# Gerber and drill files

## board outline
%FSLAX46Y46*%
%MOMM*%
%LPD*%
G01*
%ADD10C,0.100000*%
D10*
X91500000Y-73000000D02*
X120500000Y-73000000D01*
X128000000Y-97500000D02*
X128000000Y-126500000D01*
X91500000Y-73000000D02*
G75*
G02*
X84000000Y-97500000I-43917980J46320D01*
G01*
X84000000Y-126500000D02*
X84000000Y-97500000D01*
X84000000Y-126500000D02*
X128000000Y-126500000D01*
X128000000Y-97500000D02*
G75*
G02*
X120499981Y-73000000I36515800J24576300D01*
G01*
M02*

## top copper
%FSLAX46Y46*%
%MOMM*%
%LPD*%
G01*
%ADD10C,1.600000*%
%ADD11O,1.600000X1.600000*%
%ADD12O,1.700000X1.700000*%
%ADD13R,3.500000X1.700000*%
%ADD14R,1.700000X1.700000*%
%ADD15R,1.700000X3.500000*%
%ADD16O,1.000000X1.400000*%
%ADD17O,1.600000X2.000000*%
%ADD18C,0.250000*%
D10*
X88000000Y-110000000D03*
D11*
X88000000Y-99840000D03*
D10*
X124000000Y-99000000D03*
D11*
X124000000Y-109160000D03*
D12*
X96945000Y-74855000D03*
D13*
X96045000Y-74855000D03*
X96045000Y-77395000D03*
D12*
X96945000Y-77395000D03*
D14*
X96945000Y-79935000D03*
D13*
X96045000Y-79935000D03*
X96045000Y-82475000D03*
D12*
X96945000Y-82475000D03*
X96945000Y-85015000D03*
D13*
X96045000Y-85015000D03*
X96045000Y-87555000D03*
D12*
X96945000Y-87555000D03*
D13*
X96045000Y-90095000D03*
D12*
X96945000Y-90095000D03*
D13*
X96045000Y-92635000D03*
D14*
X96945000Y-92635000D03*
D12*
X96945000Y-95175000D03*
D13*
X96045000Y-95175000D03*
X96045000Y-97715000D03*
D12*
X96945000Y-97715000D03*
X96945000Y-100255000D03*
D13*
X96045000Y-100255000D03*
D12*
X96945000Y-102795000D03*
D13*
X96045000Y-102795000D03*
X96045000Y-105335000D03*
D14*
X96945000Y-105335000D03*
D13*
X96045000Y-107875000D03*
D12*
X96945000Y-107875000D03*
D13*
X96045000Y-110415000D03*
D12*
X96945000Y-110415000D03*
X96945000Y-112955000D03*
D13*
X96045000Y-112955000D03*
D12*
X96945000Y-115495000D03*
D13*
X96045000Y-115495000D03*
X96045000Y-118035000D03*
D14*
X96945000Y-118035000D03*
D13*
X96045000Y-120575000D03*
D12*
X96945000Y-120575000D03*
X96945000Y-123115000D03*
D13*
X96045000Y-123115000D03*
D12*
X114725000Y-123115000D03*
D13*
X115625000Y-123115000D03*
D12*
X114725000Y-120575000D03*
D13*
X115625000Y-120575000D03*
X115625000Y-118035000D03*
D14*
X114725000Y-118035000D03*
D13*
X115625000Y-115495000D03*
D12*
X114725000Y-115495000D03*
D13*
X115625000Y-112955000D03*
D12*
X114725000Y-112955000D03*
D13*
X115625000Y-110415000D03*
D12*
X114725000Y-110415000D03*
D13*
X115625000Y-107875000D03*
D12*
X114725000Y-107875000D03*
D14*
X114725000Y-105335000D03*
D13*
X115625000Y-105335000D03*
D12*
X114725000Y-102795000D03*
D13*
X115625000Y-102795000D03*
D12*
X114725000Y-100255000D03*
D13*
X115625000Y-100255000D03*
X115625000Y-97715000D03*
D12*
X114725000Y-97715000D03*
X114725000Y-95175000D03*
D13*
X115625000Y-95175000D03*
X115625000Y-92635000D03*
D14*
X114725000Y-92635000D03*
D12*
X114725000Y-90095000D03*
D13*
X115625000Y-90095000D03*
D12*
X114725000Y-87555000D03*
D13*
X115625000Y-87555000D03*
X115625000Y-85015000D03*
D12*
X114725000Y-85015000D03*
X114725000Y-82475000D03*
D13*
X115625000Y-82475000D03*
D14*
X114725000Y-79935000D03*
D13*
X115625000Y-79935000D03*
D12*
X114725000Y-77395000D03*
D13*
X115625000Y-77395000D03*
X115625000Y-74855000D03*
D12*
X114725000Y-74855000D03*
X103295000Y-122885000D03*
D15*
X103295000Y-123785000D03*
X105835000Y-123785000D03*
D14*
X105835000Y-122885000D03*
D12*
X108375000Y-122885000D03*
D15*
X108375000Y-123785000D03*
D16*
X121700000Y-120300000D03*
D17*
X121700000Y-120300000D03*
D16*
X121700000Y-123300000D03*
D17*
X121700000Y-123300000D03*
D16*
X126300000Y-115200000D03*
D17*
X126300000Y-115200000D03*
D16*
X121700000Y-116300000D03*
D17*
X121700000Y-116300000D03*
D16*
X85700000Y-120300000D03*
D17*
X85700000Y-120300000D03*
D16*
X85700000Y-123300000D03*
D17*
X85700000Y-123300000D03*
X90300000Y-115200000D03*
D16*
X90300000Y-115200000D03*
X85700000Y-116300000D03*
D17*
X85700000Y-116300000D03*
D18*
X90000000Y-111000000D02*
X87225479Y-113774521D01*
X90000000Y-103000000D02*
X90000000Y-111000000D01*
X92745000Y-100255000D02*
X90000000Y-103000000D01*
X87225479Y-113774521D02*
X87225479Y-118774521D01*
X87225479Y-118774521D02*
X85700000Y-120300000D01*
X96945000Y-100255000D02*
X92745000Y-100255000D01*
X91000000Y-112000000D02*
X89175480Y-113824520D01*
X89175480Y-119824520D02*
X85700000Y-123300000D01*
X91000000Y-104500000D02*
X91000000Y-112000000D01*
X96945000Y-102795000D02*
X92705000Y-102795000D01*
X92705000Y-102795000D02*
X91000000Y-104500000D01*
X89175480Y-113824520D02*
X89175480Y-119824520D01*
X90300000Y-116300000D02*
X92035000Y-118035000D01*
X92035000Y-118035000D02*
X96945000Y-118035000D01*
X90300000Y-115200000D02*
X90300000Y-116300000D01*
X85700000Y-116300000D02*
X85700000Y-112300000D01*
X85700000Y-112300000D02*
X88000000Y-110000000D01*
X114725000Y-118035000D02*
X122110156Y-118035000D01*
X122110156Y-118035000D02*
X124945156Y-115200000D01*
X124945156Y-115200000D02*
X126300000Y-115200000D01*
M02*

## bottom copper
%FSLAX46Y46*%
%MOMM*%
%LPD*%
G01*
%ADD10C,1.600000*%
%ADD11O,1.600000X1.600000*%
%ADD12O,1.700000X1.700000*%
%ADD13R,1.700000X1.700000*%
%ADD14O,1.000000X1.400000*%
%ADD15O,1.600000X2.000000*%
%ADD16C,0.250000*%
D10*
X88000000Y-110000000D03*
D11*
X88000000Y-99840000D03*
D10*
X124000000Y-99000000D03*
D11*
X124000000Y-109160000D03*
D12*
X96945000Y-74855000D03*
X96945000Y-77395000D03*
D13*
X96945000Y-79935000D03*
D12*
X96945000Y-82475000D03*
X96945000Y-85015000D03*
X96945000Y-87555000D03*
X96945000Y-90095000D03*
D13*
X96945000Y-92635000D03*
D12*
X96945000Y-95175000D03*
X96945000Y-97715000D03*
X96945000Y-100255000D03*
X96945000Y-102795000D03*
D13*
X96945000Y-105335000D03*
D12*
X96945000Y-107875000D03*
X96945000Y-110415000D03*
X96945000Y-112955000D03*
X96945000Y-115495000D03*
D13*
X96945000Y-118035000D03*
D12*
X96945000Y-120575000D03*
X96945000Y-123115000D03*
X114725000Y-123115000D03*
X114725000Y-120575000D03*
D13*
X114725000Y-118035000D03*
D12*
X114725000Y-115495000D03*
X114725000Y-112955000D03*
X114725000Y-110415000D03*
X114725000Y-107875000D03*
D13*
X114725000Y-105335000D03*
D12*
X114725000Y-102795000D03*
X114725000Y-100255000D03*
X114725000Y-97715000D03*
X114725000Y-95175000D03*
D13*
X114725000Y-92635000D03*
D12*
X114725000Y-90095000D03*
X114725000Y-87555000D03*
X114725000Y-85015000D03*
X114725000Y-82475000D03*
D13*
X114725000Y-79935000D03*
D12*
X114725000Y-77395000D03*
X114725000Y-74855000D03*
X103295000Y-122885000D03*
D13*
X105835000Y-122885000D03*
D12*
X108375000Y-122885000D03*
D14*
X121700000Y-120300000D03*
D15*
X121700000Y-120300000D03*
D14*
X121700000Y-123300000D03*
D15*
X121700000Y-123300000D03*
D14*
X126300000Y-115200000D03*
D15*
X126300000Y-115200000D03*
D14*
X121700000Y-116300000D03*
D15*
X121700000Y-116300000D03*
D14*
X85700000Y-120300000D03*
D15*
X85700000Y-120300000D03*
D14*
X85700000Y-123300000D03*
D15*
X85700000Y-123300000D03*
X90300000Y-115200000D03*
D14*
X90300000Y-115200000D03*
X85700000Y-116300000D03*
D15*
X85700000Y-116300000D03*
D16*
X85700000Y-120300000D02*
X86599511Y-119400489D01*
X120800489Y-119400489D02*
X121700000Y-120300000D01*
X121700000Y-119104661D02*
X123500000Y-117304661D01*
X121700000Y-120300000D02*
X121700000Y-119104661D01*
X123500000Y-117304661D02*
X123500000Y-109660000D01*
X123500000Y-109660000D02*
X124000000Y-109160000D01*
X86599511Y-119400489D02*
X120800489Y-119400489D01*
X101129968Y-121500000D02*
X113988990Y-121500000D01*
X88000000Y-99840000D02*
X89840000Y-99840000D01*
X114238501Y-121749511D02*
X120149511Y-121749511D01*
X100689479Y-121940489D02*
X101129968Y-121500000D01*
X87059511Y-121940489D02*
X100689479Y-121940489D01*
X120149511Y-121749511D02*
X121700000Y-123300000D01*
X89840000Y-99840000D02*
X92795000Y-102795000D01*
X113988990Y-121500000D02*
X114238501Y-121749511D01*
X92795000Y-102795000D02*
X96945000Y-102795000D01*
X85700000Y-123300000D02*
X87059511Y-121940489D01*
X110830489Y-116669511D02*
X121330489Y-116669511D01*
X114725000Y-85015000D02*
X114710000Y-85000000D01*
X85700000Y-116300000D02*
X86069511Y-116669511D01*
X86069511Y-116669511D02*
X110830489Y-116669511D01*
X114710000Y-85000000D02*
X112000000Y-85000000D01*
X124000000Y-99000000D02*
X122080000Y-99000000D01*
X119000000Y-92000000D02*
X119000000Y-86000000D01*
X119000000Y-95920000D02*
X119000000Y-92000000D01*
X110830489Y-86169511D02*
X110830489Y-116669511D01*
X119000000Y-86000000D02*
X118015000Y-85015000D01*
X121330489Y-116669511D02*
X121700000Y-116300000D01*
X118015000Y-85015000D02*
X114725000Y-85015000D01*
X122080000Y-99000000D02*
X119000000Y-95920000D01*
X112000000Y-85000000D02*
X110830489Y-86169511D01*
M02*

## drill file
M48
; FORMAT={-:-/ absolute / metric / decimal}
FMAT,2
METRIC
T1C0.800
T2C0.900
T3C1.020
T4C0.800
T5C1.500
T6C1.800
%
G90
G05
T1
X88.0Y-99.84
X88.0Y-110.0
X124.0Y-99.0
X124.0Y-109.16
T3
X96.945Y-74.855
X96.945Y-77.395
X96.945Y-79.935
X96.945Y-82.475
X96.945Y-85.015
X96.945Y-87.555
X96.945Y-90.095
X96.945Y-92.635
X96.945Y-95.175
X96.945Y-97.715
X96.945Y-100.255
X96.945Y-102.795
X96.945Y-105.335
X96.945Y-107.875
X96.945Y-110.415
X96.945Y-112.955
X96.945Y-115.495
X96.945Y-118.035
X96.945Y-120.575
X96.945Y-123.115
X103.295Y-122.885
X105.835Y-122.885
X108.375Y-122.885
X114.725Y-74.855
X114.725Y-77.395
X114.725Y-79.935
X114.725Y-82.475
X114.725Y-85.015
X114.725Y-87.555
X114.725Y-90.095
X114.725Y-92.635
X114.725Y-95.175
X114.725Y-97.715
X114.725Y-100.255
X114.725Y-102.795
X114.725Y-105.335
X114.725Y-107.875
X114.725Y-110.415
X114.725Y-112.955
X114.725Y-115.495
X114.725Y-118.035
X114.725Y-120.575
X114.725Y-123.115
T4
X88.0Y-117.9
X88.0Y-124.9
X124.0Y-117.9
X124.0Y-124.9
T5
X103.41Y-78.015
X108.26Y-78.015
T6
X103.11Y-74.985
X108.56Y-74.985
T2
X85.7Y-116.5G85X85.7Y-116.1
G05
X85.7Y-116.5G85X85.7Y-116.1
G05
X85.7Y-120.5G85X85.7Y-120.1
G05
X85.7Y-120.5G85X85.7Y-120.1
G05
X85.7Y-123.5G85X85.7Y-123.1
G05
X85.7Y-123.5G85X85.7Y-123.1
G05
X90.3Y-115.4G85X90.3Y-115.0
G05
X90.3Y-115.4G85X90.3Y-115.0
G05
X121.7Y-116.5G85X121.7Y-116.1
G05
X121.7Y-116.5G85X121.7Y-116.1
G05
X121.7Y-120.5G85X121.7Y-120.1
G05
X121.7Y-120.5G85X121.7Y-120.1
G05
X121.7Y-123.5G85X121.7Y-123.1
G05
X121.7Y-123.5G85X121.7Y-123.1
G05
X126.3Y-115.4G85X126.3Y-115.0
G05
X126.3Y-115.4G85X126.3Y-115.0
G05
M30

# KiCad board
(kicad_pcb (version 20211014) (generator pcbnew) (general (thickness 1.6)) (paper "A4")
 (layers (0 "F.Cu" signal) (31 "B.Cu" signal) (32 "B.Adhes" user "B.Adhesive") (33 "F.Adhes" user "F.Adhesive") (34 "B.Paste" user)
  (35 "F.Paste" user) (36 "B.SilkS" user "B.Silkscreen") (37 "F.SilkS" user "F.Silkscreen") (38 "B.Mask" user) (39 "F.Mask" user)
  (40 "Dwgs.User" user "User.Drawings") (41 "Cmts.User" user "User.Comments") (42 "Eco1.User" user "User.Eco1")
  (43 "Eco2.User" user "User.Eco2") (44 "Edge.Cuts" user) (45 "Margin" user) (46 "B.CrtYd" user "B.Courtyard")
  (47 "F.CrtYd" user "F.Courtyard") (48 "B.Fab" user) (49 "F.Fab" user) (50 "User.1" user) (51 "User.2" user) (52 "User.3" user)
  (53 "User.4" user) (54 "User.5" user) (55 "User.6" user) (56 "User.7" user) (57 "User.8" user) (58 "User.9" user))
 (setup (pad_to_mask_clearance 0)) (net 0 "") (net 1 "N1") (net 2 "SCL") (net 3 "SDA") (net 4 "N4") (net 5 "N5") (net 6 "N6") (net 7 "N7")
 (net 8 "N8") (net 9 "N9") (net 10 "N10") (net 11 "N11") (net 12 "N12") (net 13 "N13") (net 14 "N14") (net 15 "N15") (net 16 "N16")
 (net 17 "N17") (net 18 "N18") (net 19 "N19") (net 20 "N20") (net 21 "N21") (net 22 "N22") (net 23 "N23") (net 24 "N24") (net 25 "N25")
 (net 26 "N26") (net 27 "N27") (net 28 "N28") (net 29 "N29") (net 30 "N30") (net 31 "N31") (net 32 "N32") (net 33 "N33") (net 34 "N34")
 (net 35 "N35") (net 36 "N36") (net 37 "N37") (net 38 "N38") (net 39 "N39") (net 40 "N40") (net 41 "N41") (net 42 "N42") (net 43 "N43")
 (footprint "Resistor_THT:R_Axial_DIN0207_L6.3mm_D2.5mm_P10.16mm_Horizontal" (layer "F.Cu") (at 88 110 90)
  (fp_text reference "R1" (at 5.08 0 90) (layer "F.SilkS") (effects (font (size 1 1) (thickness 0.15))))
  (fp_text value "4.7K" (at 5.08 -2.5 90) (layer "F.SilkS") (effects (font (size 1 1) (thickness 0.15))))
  (pad "1" thru_hole circle (at 0 0 90) (size 1.6 1.6) (drill 0.8) (layers *.Cu *.Mask) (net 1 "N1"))
  (pad "2" thru_hole oval (at 10.16 0 90) (size 1.6 1.6) (drill 0.8) (layers *.Cu *.Mask) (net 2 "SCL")))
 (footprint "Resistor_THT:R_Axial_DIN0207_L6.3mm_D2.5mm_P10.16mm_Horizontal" (layer "F.Cu") (at 124 99 -90)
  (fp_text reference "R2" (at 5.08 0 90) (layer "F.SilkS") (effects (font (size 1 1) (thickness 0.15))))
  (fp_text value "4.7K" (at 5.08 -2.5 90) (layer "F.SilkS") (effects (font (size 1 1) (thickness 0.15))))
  (pad "1" thru_hole circle (at 0 0 270) (size 1.6 1.6) (drill 0.8) (layers *.Cu *.Mask) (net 1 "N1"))
  (pad "2" thru_hole oval (at 10.16 0 270) (size 1.6 1.6) (drill 0.8) (layers *.Cu *.Mask) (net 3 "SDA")))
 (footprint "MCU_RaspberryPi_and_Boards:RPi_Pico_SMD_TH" (layer "F.Cu") (at 105.835 98.985)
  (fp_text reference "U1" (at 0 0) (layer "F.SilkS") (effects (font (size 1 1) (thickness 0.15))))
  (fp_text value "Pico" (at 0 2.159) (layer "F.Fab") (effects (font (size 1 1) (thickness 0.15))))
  (pad "" np_thru_hole oval (at 2.725 -24) (size 1.8 1.8) (drill 1.8) (layers *.Cu *.Mask))
  (pad "" np_thru_hole oval (at -2.725 -24) (size 1.8 1.8) (drill 1.8) (layers *.Cu *.Mask))
  (pad "" np_thru_hole oval (at -2.425 -20.97) (size 1.5 1.5) (drill 1.5) (layers *.Cu *.Mask))
  (pad "" np_thru_hole oval (at 2.425 -20.97) (size 1.5 1.5) (drill 1.5) (layers *.Cu *.Mask))
  (pad "1" thru_hole oval (at -8.89 -24.13) (size 1.7 1.7) (drill 1.02) (layers *.Cu *.Mask) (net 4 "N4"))
  (pad "1" smd rect (at -8.89 -24.13) (size 3.5 1.7) (drill (offset -0.9 0)) (layers "F.Cu" "F.Mask") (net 4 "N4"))
  (pad "2" smd rect (at -8.89 -21.59) (size 3.5 1.7) (drill (offset -0.9 0)) (layers "F.Cu" "F.Mask") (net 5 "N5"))
  (pad "2" thru_hole oval (at -8.89 -21.59) (size 1.7 1.7) (drill 1.02) (layers *.Cu *.Mask) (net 5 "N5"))
  (pad "3" thru_hole rect (at -8.89 -19.05) (size 1.7 1.7) (drill 1.02) (layers *.Cu *.Mask) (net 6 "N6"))
  (pad "3" smd rect (at -8.89 -19.05) (size 3.5 1.7) (drill (offset -0.9 0)) (layers "F.Cu" "F.Mask") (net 6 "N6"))
  (pad "4" smd rect (at -8.89 -16.51) (size 3.5 1.7) (drill (offset -0.9 0)) (layers "F.Cu" "F.Mask") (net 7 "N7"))
  (pad "4" thru_hole oval (at -8.89 -16.51) (size 1.7 1.7) (drill 1.02) (layers *.Cu *.Mask) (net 7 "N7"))
  (pad "5" thru_hole oval (at -8.89 -13.97) (size 1.7 1.7) (drill 1.02) (layers *.Cu *.Mask) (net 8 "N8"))
  (pad "5" smd rect (at -8.89 -13.97) (size 3.5 1.7) (drill (offset -0.9 0)) (layers "F.Cu" "F.Mask") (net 8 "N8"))
  (pad "6" smd rect (at -8.89 -11.43) (size 3.5 1.7) (drill (offset -0.9 0)) (layers "F.Cu" "F.Mask") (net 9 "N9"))
  (pad "6" thru_hole oval (at -8.89 -11.43) (size 1.7 1.7) (drill 1.02) (layers *.Cu *.Mask) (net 9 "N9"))
  (pad "7" smd rect (at -8.89 -8.89) (size 3.5 1.7) (drill (offset -0.9 0)) (layers "F.Cu" "F.Mask") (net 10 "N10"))
  (pad "7" thru_hole oval (at -8.89 -8.89) (size 1.7 1.7) (drill 1.02) (layers *.Cu *.Mask) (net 10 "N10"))
  (pad "8" smd rect (at -8.89 -6.35) (size 3.5 1.7) (drill (offset -0.9 0)) (layers "F.Cu" "F.Mask") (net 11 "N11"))
  (pad "8" thru_hole rect (at -8.89 -6.35) (size 1.7 1.7) (drill 1.02) (layers *.Cu *.Mask) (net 11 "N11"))
  (pad "9" thru_hole oval (at -8.89 -3.81) (size 1.7 1.7) (drill 1.02) (layers *.Cu *.Mask) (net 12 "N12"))
  (pad "9" smd rect (at -8.89 -3.81) (size 3.5 1.7) (drill (offset -0.9 0)) (layers "F.Cu" "F.Mask") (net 12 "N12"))
  (pad "10" smd rect (at -8.89 -1.27) (size 3.5 1.7) (drill (offset -0.9 0)) (layers "F.Cu" "F.Mask") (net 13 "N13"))
  (pad "10" thru_hole oval (at -8.89 -1.27) (size 1.7 1.7) (drill 1.02) (layers *.Cu *.Mask) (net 13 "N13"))
  (pad "11" thru_hole oval (at -8.89 1.27) (size 1.7 1.7) (drill 1.02) (layers *.Cu *.Mask) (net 3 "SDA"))
  (pad "11" smd rect (at -8.89 1.27) (size 3.5 1.7) (drill (offset -0.9 0)) (layers "F.Cu" "F.Mask") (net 3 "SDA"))
  (pad "12" thru_hole oval (at -8.89 3.81) (size 1.7 1.7) (drill 1.02) (layers *.Cu *.Mask) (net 2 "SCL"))
  (pad "12" smd rect (at -8.89 3.81) (size 3.5 1.7) (drill (offset -0.9 0)) (layers "F.Cu" "F.Mask") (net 2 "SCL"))
  (pad "13" smd rect (at -8.89 6.35) (size 3.5 1.7) (drill (offset -0.9 0)) (layers "F.Cu" "F.Mask") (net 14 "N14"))
  (pad "13" thru_hole rect (at -8.89 6.35) (size 1.7 1.7) (drill 1.02) (layers *.Cu *.Mask) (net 14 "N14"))
  (pad "14" smd rect (at -8.89 8.89) (size 3.5 1.7) (drill (offset -0.9 0)) (layers "F.Cu" "F.Mask") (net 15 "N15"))
  (pad "14" thru_hole oval (at -8.89 8.89) (size 1.7 1.7) (drill 1.02) (layers *.Cu *.Mask) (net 15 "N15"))
  (pad "15" smd rect (at -8.89 11.43) (size 3.5 1.7) (drill (offset -0.9 0)) (layers "F.Cu" "F.Mask") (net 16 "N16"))
  (pad "15" thru_hole oval (at -8.89 11.43) (size 1.7 1.7) (drill 1.02) (layers *.Cu *.Mask) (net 16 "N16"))
  (pad "16" thru_hole oval (at -8.89 13.97) (size 1.7 1.7) (drill 1.02) (layers *.Cu *.Mask) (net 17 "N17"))
  (pad "16" smd rect (at -8.89 13.97) (size 3.5 1.7) (drill (offset -0.9 0)) (layers "F.Cu" "F.Mask") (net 17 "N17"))
  (pad "17" thru_hole oval (at -8.89 16.51) (size 1.7 1.7) (drill 1.02) (layers *.Cu *.Mask) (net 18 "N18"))
  (pad "17" smd rect (at -8.89 16.51) (size 3.5 1.7) (drill (offset -0.9 0)) (layers "F.Cu" "F.Mask") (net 18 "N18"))
  (pad "18" smd rect (at -8.89 19.05) (size 3.5 1.7) (drill (offset -0.9 0)) (layers "F.Cu" "F.Mask") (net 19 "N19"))
  (pad "18" thru_hole rect (at -8.89 19.05) (size 1.7 1.7) (drill 1.02) (layers *.Cu *.Mask) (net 19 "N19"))
  (pad "19" smd rect (at -8.89 21.59) (size 3.5 1.7) (drill (offset -0.9 0)) (layers "F.Cu" "F.Mask") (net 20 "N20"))
  (pad "19" thru_hole oval (at -8.89 21.59) (size 1.7 1.7) (drill 1.02) (layers *.Cu *.Mask) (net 20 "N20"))
  (pad "20" thru_hole oval (at -8.89 24.13) (size 1.7 1.7) (drill 1.02) (layers *.Cu *.Mask) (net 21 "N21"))
  (pad "20" smd rect (at -8.89 24.13) (size 3.5 1.7) (drill (offset -0.9 0)) (layers "F.Cu" "F.Mask") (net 21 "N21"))
  (pad "21" thru_hole oval (at 8.89 24.13) (size 1.7 1.7) (drill 1.02) (layers *.Cu *.Mask) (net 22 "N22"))
  (pad "21" smd rect (at 8.89 24.13) (size 3.5 1.7) (drill (offset 0.9 0)) (layers "F.Cu" "F.Mask") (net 22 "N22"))
  (pad "22" thru_hole oval (at 8.89 21.59) (size 1.7 1.7) (drill 1.02) (layers *.Cu *.Mask) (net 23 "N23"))
  (pad "22" smd rect (at 8.89 21.59) (size 3.5 1.7) (drill (offset 0.9 0)) (layers "F.Cu" "F.Mask") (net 23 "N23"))
  (pad "23" smd rect (at 8.89 19.05) (size 3.5 1.7) (drill (offset 0.9 0)) (layers "F.Cu" "F.Mask") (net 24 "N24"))
  (pad "23" thru_hole rect (at 8.89 19.05) (size 1.7 1.7) (drill 1.02) (layers *.Cu *.Mask) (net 24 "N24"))
  (pad "24" smd rect (at 8.89 16.51) (size 3.5 1.7) (drill (offset 0.9 0)) (layers "F.Cu" "F.Mask") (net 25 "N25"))
  (pad "24" thru_hole oval (at 8.89 16.51) (size 1.7 1.7) (drill 1.02) (layers *.Cu *.Mask) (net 25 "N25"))
  (pad "25" smd rect (at 8.89 13.97) (size 3.5 1.7) (drill (offset 0.9 0)) (layers "F.Cu" "F.Mask") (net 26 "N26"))
  (pad "25" thru_hole oval (at 8.89 13.97) (size 1.7 1.7) (drill 1.02) (layers *.Cu *.Mask) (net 26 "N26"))
  (pad "26" smd rect (at 8.89 11.43) (size 3.5 1.7) (drill (offset 0.9 0)) (layers "F.Cu" "F.Mask") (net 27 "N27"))
  (pad "26" thru_hole oval (at 8.89 11.43) (size 1.7 1.7) (drill 1.02) (layers *.Cu *.Mask) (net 27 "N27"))
  (pad "27" smd rect (at 8.89 8.89) (size 3.5 1.7) (drill (offset 0.9 0)) (layers "F.Cu" "F.Mask") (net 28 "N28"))
  (pad "27" thru_hole oval (at 8.89 8.89) (size 1.7 1.7) (drill 1.02) (layers *.Cu *.Mask) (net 28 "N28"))
  (pad "28" thru_hole rect (at 8.89 6.35) (size 1.7 1.7) (drill 1.02) (layers *.Cu *.Mask) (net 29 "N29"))
  (pad "28" smd rect (at 8.89 6.35) (size 3.5 1.7) (drill (offset 0.9 0)) (layers "F.Cu" "F.Mask") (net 29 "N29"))
  (pad "29" thru_hole oval (at 8.89 3.81) (size 1.7 1.7) (drill 1.02) (layers *.Cu *.Mask) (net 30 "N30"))
  (pad "29" smd rect (at 8.89 3.81) (size 3.5 1.7) (drill (offset 0.9 0)) (layers "F.Cu" "F.Mask") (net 30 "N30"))
  (pad "30" thru_hole oval (at 8.89 1.27) (size 1.7 1.7) (drill 1.02) (layers *.Cu *.Mask) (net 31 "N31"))
  (pad "30" smd rect (at 8.89 1.27) (size 3.5 1.7) (drill (offset 0.9 0)) (layers "F.Cu" "F.Mask") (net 31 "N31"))
  (pad "31" smd rect (at 8.89 -1.27) (size 3.5 1.7) (drill (offset 0.9 0)) (layers "F.Cu" "F.Mask") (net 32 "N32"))
  (pad "31" thru_hole oval (at 8.89 -1.27) (size 1.7 1.7) (drill 1.02) (layers *.Cu *.Mask) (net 32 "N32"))
  (pad "32" thru_hole oval (at 8.89 -3.81) (size 1.7 1.7) (drill 1.02) (layers *.Cu *.Mask) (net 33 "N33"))
  (pad "32" smd rect (at 8.89 -3.81) (size 3.5 1.7) (drill (offset 0.9 0)) (layers "F.Cu" "F.Mask") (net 33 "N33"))
  (pad "33" smd rect (at 8.89 -6.35) (size 3.5 1.7) (drill (offset 0.9 0)) (layers "F.Cu" "F.Mask") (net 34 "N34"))
  (pad "33" thru_hole rect (at 8.89 -6.35) (size 1.7 1.7) (drill 1.02) (layers *.Cu *.Mask) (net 34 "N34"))
  (pad "34" thru_hole oval (at 8.89 -8.89) (size 1.7 1.7) (drill 1.02) (layers *.Cu *.Mask) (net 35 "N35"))
  (pad "34" smd rect (at 8.89 -8.89) (size 3.5 1.7) (drill (offset 0.9 0)) (layers "F.Cu" "F.Mask") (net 35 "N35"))
  (pad "35" thru_hole oval (at 8.89 -11.43) (size 1.7 1.7) (drill 1.02) (layers *.Cu *.Mask) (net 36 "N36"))
  (pad "35" smd rect (at 8.89 -11.43) (size 3.5 1.7) (drill (offset 0.9 0)) (layers "F.Cu" "F.Mask") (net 36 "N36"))
  (pad "36" smd rect (at 8.89 -13.97) (size 3.5 1.7) (drill (offset 0.9 0)) (layers "F.Cu" "F.Mask") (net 1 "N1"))
  (pad "36" thru_hole oval (at 8.89 -13.97) (size 1.7 1.7) (drill 1.02) (layers *.Cu *.Mask) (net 1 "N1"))
  (pad "37" thru_hole oval (at 8.89 -16.51) (size 1.7 1.7) (drill 1.02) (layers *.Cu *.Mask) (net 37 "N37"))
  (pad "37" smd rect (at 8.89 -16.51) (size 3.5 1.7) (drill (offset 0.9 0)) (layers "F.Cu" "F.Mask") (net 37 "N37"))
  (pad "38" thru_hole rect (at 8.89 -19.05) (size 1.7 1.7) (drill 1.02) (layers *.Cu *.Mask) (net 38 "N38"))
  (pad "38" smd rect (at 8.89 -19.05) (size 3.5 1.7) (drill (offset 0.9 0)) (layers "F.Cu" "F.Mask") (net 38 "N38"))
  (pad "39" thru_hole oval (at 8.89 -21.59) (size 1.7 1.7) (drill 1.02) (layers *.Cu *.Mask) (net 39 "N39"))
  (pad "39" smd rect (at 8.89 -21.59) (size 3.5 1.7) (drill (offset 0.9 0)) (layers "F.Cu" "F.Mask") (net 39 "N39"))
  (pad "40" smd rect (at 8.89 -24.13) (size 3.5 1.7) (drill (offset 0.9 0)) (layers "F.Cu" "F.Mask") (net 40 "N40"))
  (pad "40" thru_hole oval (at 8.89 -24.13) (size 1.7 1.7) (drill 1.02) (layers *.Cu *.Mask) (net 40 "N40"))
  (pad "41" thru_hole oval (at -2.54 23.9) (size 1.7 1.7) (drill 1.02) (layers *.Cu *.Mask) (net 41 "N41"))
  (pad "41" smd rect (at -2.54 23.9 90) (size 3.5 1.7) (drill (offset -0.9 0)) (layers "F.Cu" "F.Mask") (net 41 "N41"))
  (pad "42" smd rect (at 0 23.9 90) (size 3.5 1.7) (drill (offset -0.9 0)) (layers "F.Cu" "F.Mask") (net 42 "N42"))
  (pad "42" thru_hole rect (at 0 23.9) (size 1.7 1.7) (drill 1.02) (layers *.Cu *.Mask) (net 42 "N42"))
  (pad "43" thru_hole oval (at 2.54 23.9) (size 1.7 1.7) (drill 1.02) (layers *.Cu *.Mask) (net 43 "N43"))
  (pad "43" smd rect (at 2.54 23.9 90) (size 3.5 1.7) (drill (offset -0.9 0)) (layers "F.Cu" "F.Mask") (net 43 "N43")))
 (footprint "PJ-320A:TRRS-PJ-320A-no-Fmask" (layer "F.Cu") (at 124 126.5 180)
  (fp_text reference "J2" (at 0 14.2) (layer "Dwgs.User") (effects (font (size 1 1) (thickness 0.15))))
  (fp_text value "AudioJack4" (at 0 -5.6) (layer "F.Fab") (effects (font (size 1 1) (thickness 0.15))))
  (pad "" np_thru_hole circle (at 0 1.6 180) (size 0.8 0.8) (drill 0.8) (layers *.Cu *.Mask))
  (pad "" np_thru_hole circle (at 0 8.6 180) (size 0.8 0.8) (drill 0.8) (layers *.Cu *.Mask))
  (pad "R1" thru_hole oval (at 2.3 6.2 180) (size 1 1.4) (drill oval 0.9 1.3) (layers *.Cu "F.Mask") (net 3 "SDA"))
  (pad "R1" thru_hole oval (at 2.3 6.2 180) (size 1.6 2) (drill oval 0.9 1.3) (layers *.Cu "B.Mask") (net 3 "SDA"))
  (pad "R2" thru_hole oval (at 2.3 3.2 180) (size 1 1.4) (drill oval 0.9 1.3) (layers *.Cu "F.Mask") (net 2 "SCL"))
  (pad "R2" thru_hole oval (at 2.3 3.2 180) (size 1.6 2) (drill oval 0.9 1.3) (layers *.Cu "B.Mask") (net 2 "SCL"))
  (pad "S" thru_hole oval (at -2.3 11.3 180) (size 1 1.4) (drill oval 0.9 1.3) (layers *.Cu "F.Mask") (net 24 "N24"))
  (pad "S" thru_hole oval (at -2.3 11.3 180) (size 1.6 2) (drill oval 0.9 1.3) (layers *.Cu "B.Mask") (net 24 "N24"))
  (pad "T" thru_hole oval (at 2.3 10.2 180) (size 1 1.4) (drill oval 0.9 1.3) (layers *.Cu "F.Mask") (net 1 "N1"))
  (pad "T" thru_hole oval (at 2.3 10.2 180) (size 1.6 2) (drill oval 0.9 1.3) (layers *.Cu "B.Mask") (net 1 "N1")))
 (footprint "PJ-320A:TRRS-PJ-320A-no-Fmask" (layer "F.Cu") (at 88 126.5 180)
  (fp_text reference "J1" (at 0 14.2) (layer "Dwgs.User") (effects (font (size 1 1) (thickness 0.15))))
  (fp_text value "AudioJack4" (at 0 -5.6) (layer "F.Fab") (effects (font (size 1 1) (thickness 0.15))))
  (pad "" np_thru_hole circle (at 0 8.6 180) (size 0.8 0.8) (drill 0.8) (layers *.Cu *.Mask))
  (pad "" np_thru_hole circle (at 0 1.6 180) (size 0.8 0.8) (drill 0.8) (layers *.Cu *.Mask))
  (pad "R1" thru_hole oval (at 2.3 6.2 180) (size 1 1.4) (drill oval 0.9 1.3) (layers *.Cu "F.Mask") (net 3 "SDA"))
  (pad "R1" thru_hole oval (at 2.3 6.2 180) (size 1.6 2) (drill oval 0.9 1.3) (layers *.Cu "B.Mask") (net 3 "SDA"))
  (pad "R2" thru_hole oval (at 2.3 3.2 180) (size 1 1.4) (drill oval 0.9 1.3) (layers *.Cu "F.Mask") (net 2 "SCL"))
  (pad "R2" thru_hole oval (at 2.3 3.2 180) (size 1.6 2) (drill oval 0.9 1.3) (layers *.Cu "B.Mask") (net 2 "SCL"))
  (pad "S" thru_hole oval (at -2.3 11.3 180) (size 1.6 2) (drill oval 0.9 1.3) (layers *.Cu "B.Mask") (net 19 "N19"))
  (pad "S" thru_hole oval (at -2.3 11.3 180) (size 1 1.4) (drill oval 0.9 1.3) (layers *.Cu "F.Mask") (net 19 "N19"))
  (pad "T" thru_hole oval (at 2.3 10.2 180) (size 1 1.4) (drill oval 0.9 1.3) (layers *.Cu "F.Mask") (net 1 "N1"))
  (pad "T" thru_hole oval (at 2.3 10.2 180) (size 1.6 2) (drill oval 0.9 1.3) (layers *.Cu "B.Mask") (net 1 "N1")))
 (gr_line (start 91.5 73) (end 120.5 73) (layer "Edge.Cuts") (width 0.1))
 (gr_line (start 128 97.5) (end 128 126.5) (layer "Edge.Cuts") (width 0.1))
 (gr_arc (start 91.5 73) (mid 89.576413 85.809109) (end 84 97.5) (layer "Edge.Cuts") (width 0.1))
 (gr_line (start 84 126.5) (end 84 97.5) (layer "Edge.Cuts") (width 0.1))
 (gr_line (start 84 126.5) (end 128 126.5) (layer "Edge.Cuts") (width 0.1))
 (gr_arc (start 128 97.5) (mid 122.427832 85.80781) (end 120.5 73) (layer "Edge.Cuts") (width 0.1))
 (segment (start 90 111) (end 87.225479 113.774521) (width 0.25) (layer "F.Cu") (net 3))
 (segment (start 90 103) (end 90 111) (width 0.25) (layer "F.Cu") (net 3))
 (segment (start 92.745 100.255) (end 90 103) (width 0.25) (layer "F.Cu") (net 3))
 (segment (start 87.225479 113.774521) (end 87.225479 118.774521) (width 0.25) (layer "F.Cu") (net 3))
 (segment (start 87.225479 118.774521) (end 85.7 120.3) (width 0.25) (layer "F.Cu") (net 3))
 (segment (start 96.945 100.255) (end 92.745 100.255) (width 0.25) (layer "F.Cu") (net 3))
 (segment (start 85.7 120.3) (end 86.599511 119.400489) (width 0.25) (layer "B.Cu") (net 3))
 (segment (start 120.800489 119.400489) (end 121.7 120.3) (width 0.25) (layer "B.Cu") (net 3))
 (segment (start 121.7 119.104661) (end 123.5 117.304661) (width 0.25) (layer "B.Cu") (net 3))
 (segment (start 121.7 120.3) (end 121.7 119.104661) (width 0.25) (layer "B.Cu") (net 3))
 (segment (start 123.5 117.304661) (end 123.5 109.66) (width 0.25) (layer "B.Cu") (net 3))
 (segment (start 123.5 109.66) (end 124 109.16) (width 0.25) (layer "B.Cu") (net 3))
 (segment (start 86.599511 119.400489) (end 120.800489 119.400489) (width 0.25) (layer "B.Cu") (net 3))
 (segment (start 91 112) (end 89.17548 113.82452) (width 0.25) (layer "F.Cu") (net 2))
 (segment (start 89.17548 119.82452) (end 85.7 123.3) (width 0.25) (layer "F.Cu") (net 2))
 (segment (start 91 104.5) (end 91 112) (width 0.25) (layer "F.Cu") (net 2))
 (segment (start 96.945 102.795) (end 92.705 102.795) (width 0.25) (layer "F.Cu") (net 2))
 (segment (start 92.705 102.795) (end 91 104.5) (width 0.25) (layer "F.Cu") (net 2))
 (segment (start 89.17548 113.82452) (end 89.17548 119.82452) (width 0.25) (layer "F.Cu") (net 2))
 (segment (start 101.129968 121.5) (end 113.98899 121.5) (width 0.25) (layer "B.Cu") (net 2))
 (segment (start 88 99.84) (end 89.84 99.84) (width 0.25) (layer "B.Cu") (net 2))
 (segment (start 114.238501 121.749511) (end 120.149511 121.749511) (width 0.25) (layer "B.Cu") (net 2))
 (segment (start 100.689479 121.940489) (end 101.129968 121.5) (width 0.25) (layer "B.Cu") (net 2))
 (segment (start 87.059511 121.940489) (end 100.689479 121.940489) (width 0.25) (layer "B.Cu") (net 2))
 (segment (start 120.149511 121.749511) (end 121.7 123.3) (width 0.25) (layer "B.Cu") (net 2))
 (segment (start 89.84 99.84) (end 92.795 102.795) (width 0.25) (layer "B.Cu") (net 2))
 (segment (start 113.98899 121.5) (end 114.238501 121.749511) (width 0.25) (layer "B.Cu") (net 2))
 (segment (start 92.795 102.795) (end 96.945 102.795) (width 0.25) (layer "B.Cu") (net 2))
 (segment (start 85.7 123.3) (end 87.059511 121.940489) (width 0.25) (layer "B.Cu") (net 2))
 (segment (start 90.3 116.3) (end 92.035 118.035) (width 0.25) (layer "F.Cu") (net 19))
 (segment (start 92.035 118.035) (end 96.945 118.035) (width 0.25) (layer "F.Cu") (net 19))
 (segment (start 90.3 115.2) (end 90.3 116.3) (width 0.25) (layer "F.Cu") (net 19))
 (segment (start 85.7 116.3) (end 85.7 112.3) (width 0.25) (layer "F.Cu") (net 1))
 (segment (start 85.7 112.3) (end 88 110) (width 0.25) (layer "F.Cu") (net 1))
 (segment (start 110.830489 116.669511) (end 121.330489 116.669511) (width 0.25) (layer "B.Cu") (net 1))
 (segment (start 114.725 85.015) (end 114.71 85) (width 0.25) (layer "B.Cu") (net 1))
 (segment (start 85.7 116.3) (end 86.069511 116.669511) (width 0.25) (layer "B.Cu") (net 1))
 (segment (start 86.069511 116.669511) (end 110.830489 116.669511) (width 0.25) (layer "B.Cu") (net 1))
 (segment (start 114.71 85) (end 112 85) (width 0.25) (layer "B.Cu") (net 1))
 (segment (start 124 99) (end 122.08 99) (width 0.25) (layer "B.Cu") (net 1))
 (segment (start 119 92) (end 119 86) (width 0.25) (layer "B.Cu") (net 1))
 (segment (start 119 95.92) (end 119 92) (width 0.25) (layer "B.Cu") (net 1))
 (segment (start 110.830489 86.169511) (end 110.830489 116.669511) (width 0.25) (layer "B.Cu") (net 1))
 (segment (start 119 86) (end 118.015 85.015) (width 0.25) (layer "B.Cu") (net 1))
 (segment (start 121.330489 116.669511) (end 121.7 116.3) (width 0.25) (layer "B.Cu") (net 1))
 (segment (start 118.015 85.015) (end 114.725 85.015) (width 0.25) (layer "B.Cu") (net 1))
 (segment (start 122.08 99) (end 119 95.92) (width 0.25) (layer "B.Cu") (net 1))
 (segment (start 112 85) (end 110.830489 86.169511) (width 0.25) (layer "B.Cu") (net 1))
 (segment (start 114.725 118.035) (end 122.110156 118.035) (width 0.25) (layer "F.Cu") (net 24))
 (segment (start 122.110156 118.035) (end 124.945156 115.2) (width 0.25) (layer "F.Cu") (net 24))
 (segment (start 124.945156 115.2) (end 126.3 115.2) (width 0.25) (layer "F.Cu") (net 24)))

